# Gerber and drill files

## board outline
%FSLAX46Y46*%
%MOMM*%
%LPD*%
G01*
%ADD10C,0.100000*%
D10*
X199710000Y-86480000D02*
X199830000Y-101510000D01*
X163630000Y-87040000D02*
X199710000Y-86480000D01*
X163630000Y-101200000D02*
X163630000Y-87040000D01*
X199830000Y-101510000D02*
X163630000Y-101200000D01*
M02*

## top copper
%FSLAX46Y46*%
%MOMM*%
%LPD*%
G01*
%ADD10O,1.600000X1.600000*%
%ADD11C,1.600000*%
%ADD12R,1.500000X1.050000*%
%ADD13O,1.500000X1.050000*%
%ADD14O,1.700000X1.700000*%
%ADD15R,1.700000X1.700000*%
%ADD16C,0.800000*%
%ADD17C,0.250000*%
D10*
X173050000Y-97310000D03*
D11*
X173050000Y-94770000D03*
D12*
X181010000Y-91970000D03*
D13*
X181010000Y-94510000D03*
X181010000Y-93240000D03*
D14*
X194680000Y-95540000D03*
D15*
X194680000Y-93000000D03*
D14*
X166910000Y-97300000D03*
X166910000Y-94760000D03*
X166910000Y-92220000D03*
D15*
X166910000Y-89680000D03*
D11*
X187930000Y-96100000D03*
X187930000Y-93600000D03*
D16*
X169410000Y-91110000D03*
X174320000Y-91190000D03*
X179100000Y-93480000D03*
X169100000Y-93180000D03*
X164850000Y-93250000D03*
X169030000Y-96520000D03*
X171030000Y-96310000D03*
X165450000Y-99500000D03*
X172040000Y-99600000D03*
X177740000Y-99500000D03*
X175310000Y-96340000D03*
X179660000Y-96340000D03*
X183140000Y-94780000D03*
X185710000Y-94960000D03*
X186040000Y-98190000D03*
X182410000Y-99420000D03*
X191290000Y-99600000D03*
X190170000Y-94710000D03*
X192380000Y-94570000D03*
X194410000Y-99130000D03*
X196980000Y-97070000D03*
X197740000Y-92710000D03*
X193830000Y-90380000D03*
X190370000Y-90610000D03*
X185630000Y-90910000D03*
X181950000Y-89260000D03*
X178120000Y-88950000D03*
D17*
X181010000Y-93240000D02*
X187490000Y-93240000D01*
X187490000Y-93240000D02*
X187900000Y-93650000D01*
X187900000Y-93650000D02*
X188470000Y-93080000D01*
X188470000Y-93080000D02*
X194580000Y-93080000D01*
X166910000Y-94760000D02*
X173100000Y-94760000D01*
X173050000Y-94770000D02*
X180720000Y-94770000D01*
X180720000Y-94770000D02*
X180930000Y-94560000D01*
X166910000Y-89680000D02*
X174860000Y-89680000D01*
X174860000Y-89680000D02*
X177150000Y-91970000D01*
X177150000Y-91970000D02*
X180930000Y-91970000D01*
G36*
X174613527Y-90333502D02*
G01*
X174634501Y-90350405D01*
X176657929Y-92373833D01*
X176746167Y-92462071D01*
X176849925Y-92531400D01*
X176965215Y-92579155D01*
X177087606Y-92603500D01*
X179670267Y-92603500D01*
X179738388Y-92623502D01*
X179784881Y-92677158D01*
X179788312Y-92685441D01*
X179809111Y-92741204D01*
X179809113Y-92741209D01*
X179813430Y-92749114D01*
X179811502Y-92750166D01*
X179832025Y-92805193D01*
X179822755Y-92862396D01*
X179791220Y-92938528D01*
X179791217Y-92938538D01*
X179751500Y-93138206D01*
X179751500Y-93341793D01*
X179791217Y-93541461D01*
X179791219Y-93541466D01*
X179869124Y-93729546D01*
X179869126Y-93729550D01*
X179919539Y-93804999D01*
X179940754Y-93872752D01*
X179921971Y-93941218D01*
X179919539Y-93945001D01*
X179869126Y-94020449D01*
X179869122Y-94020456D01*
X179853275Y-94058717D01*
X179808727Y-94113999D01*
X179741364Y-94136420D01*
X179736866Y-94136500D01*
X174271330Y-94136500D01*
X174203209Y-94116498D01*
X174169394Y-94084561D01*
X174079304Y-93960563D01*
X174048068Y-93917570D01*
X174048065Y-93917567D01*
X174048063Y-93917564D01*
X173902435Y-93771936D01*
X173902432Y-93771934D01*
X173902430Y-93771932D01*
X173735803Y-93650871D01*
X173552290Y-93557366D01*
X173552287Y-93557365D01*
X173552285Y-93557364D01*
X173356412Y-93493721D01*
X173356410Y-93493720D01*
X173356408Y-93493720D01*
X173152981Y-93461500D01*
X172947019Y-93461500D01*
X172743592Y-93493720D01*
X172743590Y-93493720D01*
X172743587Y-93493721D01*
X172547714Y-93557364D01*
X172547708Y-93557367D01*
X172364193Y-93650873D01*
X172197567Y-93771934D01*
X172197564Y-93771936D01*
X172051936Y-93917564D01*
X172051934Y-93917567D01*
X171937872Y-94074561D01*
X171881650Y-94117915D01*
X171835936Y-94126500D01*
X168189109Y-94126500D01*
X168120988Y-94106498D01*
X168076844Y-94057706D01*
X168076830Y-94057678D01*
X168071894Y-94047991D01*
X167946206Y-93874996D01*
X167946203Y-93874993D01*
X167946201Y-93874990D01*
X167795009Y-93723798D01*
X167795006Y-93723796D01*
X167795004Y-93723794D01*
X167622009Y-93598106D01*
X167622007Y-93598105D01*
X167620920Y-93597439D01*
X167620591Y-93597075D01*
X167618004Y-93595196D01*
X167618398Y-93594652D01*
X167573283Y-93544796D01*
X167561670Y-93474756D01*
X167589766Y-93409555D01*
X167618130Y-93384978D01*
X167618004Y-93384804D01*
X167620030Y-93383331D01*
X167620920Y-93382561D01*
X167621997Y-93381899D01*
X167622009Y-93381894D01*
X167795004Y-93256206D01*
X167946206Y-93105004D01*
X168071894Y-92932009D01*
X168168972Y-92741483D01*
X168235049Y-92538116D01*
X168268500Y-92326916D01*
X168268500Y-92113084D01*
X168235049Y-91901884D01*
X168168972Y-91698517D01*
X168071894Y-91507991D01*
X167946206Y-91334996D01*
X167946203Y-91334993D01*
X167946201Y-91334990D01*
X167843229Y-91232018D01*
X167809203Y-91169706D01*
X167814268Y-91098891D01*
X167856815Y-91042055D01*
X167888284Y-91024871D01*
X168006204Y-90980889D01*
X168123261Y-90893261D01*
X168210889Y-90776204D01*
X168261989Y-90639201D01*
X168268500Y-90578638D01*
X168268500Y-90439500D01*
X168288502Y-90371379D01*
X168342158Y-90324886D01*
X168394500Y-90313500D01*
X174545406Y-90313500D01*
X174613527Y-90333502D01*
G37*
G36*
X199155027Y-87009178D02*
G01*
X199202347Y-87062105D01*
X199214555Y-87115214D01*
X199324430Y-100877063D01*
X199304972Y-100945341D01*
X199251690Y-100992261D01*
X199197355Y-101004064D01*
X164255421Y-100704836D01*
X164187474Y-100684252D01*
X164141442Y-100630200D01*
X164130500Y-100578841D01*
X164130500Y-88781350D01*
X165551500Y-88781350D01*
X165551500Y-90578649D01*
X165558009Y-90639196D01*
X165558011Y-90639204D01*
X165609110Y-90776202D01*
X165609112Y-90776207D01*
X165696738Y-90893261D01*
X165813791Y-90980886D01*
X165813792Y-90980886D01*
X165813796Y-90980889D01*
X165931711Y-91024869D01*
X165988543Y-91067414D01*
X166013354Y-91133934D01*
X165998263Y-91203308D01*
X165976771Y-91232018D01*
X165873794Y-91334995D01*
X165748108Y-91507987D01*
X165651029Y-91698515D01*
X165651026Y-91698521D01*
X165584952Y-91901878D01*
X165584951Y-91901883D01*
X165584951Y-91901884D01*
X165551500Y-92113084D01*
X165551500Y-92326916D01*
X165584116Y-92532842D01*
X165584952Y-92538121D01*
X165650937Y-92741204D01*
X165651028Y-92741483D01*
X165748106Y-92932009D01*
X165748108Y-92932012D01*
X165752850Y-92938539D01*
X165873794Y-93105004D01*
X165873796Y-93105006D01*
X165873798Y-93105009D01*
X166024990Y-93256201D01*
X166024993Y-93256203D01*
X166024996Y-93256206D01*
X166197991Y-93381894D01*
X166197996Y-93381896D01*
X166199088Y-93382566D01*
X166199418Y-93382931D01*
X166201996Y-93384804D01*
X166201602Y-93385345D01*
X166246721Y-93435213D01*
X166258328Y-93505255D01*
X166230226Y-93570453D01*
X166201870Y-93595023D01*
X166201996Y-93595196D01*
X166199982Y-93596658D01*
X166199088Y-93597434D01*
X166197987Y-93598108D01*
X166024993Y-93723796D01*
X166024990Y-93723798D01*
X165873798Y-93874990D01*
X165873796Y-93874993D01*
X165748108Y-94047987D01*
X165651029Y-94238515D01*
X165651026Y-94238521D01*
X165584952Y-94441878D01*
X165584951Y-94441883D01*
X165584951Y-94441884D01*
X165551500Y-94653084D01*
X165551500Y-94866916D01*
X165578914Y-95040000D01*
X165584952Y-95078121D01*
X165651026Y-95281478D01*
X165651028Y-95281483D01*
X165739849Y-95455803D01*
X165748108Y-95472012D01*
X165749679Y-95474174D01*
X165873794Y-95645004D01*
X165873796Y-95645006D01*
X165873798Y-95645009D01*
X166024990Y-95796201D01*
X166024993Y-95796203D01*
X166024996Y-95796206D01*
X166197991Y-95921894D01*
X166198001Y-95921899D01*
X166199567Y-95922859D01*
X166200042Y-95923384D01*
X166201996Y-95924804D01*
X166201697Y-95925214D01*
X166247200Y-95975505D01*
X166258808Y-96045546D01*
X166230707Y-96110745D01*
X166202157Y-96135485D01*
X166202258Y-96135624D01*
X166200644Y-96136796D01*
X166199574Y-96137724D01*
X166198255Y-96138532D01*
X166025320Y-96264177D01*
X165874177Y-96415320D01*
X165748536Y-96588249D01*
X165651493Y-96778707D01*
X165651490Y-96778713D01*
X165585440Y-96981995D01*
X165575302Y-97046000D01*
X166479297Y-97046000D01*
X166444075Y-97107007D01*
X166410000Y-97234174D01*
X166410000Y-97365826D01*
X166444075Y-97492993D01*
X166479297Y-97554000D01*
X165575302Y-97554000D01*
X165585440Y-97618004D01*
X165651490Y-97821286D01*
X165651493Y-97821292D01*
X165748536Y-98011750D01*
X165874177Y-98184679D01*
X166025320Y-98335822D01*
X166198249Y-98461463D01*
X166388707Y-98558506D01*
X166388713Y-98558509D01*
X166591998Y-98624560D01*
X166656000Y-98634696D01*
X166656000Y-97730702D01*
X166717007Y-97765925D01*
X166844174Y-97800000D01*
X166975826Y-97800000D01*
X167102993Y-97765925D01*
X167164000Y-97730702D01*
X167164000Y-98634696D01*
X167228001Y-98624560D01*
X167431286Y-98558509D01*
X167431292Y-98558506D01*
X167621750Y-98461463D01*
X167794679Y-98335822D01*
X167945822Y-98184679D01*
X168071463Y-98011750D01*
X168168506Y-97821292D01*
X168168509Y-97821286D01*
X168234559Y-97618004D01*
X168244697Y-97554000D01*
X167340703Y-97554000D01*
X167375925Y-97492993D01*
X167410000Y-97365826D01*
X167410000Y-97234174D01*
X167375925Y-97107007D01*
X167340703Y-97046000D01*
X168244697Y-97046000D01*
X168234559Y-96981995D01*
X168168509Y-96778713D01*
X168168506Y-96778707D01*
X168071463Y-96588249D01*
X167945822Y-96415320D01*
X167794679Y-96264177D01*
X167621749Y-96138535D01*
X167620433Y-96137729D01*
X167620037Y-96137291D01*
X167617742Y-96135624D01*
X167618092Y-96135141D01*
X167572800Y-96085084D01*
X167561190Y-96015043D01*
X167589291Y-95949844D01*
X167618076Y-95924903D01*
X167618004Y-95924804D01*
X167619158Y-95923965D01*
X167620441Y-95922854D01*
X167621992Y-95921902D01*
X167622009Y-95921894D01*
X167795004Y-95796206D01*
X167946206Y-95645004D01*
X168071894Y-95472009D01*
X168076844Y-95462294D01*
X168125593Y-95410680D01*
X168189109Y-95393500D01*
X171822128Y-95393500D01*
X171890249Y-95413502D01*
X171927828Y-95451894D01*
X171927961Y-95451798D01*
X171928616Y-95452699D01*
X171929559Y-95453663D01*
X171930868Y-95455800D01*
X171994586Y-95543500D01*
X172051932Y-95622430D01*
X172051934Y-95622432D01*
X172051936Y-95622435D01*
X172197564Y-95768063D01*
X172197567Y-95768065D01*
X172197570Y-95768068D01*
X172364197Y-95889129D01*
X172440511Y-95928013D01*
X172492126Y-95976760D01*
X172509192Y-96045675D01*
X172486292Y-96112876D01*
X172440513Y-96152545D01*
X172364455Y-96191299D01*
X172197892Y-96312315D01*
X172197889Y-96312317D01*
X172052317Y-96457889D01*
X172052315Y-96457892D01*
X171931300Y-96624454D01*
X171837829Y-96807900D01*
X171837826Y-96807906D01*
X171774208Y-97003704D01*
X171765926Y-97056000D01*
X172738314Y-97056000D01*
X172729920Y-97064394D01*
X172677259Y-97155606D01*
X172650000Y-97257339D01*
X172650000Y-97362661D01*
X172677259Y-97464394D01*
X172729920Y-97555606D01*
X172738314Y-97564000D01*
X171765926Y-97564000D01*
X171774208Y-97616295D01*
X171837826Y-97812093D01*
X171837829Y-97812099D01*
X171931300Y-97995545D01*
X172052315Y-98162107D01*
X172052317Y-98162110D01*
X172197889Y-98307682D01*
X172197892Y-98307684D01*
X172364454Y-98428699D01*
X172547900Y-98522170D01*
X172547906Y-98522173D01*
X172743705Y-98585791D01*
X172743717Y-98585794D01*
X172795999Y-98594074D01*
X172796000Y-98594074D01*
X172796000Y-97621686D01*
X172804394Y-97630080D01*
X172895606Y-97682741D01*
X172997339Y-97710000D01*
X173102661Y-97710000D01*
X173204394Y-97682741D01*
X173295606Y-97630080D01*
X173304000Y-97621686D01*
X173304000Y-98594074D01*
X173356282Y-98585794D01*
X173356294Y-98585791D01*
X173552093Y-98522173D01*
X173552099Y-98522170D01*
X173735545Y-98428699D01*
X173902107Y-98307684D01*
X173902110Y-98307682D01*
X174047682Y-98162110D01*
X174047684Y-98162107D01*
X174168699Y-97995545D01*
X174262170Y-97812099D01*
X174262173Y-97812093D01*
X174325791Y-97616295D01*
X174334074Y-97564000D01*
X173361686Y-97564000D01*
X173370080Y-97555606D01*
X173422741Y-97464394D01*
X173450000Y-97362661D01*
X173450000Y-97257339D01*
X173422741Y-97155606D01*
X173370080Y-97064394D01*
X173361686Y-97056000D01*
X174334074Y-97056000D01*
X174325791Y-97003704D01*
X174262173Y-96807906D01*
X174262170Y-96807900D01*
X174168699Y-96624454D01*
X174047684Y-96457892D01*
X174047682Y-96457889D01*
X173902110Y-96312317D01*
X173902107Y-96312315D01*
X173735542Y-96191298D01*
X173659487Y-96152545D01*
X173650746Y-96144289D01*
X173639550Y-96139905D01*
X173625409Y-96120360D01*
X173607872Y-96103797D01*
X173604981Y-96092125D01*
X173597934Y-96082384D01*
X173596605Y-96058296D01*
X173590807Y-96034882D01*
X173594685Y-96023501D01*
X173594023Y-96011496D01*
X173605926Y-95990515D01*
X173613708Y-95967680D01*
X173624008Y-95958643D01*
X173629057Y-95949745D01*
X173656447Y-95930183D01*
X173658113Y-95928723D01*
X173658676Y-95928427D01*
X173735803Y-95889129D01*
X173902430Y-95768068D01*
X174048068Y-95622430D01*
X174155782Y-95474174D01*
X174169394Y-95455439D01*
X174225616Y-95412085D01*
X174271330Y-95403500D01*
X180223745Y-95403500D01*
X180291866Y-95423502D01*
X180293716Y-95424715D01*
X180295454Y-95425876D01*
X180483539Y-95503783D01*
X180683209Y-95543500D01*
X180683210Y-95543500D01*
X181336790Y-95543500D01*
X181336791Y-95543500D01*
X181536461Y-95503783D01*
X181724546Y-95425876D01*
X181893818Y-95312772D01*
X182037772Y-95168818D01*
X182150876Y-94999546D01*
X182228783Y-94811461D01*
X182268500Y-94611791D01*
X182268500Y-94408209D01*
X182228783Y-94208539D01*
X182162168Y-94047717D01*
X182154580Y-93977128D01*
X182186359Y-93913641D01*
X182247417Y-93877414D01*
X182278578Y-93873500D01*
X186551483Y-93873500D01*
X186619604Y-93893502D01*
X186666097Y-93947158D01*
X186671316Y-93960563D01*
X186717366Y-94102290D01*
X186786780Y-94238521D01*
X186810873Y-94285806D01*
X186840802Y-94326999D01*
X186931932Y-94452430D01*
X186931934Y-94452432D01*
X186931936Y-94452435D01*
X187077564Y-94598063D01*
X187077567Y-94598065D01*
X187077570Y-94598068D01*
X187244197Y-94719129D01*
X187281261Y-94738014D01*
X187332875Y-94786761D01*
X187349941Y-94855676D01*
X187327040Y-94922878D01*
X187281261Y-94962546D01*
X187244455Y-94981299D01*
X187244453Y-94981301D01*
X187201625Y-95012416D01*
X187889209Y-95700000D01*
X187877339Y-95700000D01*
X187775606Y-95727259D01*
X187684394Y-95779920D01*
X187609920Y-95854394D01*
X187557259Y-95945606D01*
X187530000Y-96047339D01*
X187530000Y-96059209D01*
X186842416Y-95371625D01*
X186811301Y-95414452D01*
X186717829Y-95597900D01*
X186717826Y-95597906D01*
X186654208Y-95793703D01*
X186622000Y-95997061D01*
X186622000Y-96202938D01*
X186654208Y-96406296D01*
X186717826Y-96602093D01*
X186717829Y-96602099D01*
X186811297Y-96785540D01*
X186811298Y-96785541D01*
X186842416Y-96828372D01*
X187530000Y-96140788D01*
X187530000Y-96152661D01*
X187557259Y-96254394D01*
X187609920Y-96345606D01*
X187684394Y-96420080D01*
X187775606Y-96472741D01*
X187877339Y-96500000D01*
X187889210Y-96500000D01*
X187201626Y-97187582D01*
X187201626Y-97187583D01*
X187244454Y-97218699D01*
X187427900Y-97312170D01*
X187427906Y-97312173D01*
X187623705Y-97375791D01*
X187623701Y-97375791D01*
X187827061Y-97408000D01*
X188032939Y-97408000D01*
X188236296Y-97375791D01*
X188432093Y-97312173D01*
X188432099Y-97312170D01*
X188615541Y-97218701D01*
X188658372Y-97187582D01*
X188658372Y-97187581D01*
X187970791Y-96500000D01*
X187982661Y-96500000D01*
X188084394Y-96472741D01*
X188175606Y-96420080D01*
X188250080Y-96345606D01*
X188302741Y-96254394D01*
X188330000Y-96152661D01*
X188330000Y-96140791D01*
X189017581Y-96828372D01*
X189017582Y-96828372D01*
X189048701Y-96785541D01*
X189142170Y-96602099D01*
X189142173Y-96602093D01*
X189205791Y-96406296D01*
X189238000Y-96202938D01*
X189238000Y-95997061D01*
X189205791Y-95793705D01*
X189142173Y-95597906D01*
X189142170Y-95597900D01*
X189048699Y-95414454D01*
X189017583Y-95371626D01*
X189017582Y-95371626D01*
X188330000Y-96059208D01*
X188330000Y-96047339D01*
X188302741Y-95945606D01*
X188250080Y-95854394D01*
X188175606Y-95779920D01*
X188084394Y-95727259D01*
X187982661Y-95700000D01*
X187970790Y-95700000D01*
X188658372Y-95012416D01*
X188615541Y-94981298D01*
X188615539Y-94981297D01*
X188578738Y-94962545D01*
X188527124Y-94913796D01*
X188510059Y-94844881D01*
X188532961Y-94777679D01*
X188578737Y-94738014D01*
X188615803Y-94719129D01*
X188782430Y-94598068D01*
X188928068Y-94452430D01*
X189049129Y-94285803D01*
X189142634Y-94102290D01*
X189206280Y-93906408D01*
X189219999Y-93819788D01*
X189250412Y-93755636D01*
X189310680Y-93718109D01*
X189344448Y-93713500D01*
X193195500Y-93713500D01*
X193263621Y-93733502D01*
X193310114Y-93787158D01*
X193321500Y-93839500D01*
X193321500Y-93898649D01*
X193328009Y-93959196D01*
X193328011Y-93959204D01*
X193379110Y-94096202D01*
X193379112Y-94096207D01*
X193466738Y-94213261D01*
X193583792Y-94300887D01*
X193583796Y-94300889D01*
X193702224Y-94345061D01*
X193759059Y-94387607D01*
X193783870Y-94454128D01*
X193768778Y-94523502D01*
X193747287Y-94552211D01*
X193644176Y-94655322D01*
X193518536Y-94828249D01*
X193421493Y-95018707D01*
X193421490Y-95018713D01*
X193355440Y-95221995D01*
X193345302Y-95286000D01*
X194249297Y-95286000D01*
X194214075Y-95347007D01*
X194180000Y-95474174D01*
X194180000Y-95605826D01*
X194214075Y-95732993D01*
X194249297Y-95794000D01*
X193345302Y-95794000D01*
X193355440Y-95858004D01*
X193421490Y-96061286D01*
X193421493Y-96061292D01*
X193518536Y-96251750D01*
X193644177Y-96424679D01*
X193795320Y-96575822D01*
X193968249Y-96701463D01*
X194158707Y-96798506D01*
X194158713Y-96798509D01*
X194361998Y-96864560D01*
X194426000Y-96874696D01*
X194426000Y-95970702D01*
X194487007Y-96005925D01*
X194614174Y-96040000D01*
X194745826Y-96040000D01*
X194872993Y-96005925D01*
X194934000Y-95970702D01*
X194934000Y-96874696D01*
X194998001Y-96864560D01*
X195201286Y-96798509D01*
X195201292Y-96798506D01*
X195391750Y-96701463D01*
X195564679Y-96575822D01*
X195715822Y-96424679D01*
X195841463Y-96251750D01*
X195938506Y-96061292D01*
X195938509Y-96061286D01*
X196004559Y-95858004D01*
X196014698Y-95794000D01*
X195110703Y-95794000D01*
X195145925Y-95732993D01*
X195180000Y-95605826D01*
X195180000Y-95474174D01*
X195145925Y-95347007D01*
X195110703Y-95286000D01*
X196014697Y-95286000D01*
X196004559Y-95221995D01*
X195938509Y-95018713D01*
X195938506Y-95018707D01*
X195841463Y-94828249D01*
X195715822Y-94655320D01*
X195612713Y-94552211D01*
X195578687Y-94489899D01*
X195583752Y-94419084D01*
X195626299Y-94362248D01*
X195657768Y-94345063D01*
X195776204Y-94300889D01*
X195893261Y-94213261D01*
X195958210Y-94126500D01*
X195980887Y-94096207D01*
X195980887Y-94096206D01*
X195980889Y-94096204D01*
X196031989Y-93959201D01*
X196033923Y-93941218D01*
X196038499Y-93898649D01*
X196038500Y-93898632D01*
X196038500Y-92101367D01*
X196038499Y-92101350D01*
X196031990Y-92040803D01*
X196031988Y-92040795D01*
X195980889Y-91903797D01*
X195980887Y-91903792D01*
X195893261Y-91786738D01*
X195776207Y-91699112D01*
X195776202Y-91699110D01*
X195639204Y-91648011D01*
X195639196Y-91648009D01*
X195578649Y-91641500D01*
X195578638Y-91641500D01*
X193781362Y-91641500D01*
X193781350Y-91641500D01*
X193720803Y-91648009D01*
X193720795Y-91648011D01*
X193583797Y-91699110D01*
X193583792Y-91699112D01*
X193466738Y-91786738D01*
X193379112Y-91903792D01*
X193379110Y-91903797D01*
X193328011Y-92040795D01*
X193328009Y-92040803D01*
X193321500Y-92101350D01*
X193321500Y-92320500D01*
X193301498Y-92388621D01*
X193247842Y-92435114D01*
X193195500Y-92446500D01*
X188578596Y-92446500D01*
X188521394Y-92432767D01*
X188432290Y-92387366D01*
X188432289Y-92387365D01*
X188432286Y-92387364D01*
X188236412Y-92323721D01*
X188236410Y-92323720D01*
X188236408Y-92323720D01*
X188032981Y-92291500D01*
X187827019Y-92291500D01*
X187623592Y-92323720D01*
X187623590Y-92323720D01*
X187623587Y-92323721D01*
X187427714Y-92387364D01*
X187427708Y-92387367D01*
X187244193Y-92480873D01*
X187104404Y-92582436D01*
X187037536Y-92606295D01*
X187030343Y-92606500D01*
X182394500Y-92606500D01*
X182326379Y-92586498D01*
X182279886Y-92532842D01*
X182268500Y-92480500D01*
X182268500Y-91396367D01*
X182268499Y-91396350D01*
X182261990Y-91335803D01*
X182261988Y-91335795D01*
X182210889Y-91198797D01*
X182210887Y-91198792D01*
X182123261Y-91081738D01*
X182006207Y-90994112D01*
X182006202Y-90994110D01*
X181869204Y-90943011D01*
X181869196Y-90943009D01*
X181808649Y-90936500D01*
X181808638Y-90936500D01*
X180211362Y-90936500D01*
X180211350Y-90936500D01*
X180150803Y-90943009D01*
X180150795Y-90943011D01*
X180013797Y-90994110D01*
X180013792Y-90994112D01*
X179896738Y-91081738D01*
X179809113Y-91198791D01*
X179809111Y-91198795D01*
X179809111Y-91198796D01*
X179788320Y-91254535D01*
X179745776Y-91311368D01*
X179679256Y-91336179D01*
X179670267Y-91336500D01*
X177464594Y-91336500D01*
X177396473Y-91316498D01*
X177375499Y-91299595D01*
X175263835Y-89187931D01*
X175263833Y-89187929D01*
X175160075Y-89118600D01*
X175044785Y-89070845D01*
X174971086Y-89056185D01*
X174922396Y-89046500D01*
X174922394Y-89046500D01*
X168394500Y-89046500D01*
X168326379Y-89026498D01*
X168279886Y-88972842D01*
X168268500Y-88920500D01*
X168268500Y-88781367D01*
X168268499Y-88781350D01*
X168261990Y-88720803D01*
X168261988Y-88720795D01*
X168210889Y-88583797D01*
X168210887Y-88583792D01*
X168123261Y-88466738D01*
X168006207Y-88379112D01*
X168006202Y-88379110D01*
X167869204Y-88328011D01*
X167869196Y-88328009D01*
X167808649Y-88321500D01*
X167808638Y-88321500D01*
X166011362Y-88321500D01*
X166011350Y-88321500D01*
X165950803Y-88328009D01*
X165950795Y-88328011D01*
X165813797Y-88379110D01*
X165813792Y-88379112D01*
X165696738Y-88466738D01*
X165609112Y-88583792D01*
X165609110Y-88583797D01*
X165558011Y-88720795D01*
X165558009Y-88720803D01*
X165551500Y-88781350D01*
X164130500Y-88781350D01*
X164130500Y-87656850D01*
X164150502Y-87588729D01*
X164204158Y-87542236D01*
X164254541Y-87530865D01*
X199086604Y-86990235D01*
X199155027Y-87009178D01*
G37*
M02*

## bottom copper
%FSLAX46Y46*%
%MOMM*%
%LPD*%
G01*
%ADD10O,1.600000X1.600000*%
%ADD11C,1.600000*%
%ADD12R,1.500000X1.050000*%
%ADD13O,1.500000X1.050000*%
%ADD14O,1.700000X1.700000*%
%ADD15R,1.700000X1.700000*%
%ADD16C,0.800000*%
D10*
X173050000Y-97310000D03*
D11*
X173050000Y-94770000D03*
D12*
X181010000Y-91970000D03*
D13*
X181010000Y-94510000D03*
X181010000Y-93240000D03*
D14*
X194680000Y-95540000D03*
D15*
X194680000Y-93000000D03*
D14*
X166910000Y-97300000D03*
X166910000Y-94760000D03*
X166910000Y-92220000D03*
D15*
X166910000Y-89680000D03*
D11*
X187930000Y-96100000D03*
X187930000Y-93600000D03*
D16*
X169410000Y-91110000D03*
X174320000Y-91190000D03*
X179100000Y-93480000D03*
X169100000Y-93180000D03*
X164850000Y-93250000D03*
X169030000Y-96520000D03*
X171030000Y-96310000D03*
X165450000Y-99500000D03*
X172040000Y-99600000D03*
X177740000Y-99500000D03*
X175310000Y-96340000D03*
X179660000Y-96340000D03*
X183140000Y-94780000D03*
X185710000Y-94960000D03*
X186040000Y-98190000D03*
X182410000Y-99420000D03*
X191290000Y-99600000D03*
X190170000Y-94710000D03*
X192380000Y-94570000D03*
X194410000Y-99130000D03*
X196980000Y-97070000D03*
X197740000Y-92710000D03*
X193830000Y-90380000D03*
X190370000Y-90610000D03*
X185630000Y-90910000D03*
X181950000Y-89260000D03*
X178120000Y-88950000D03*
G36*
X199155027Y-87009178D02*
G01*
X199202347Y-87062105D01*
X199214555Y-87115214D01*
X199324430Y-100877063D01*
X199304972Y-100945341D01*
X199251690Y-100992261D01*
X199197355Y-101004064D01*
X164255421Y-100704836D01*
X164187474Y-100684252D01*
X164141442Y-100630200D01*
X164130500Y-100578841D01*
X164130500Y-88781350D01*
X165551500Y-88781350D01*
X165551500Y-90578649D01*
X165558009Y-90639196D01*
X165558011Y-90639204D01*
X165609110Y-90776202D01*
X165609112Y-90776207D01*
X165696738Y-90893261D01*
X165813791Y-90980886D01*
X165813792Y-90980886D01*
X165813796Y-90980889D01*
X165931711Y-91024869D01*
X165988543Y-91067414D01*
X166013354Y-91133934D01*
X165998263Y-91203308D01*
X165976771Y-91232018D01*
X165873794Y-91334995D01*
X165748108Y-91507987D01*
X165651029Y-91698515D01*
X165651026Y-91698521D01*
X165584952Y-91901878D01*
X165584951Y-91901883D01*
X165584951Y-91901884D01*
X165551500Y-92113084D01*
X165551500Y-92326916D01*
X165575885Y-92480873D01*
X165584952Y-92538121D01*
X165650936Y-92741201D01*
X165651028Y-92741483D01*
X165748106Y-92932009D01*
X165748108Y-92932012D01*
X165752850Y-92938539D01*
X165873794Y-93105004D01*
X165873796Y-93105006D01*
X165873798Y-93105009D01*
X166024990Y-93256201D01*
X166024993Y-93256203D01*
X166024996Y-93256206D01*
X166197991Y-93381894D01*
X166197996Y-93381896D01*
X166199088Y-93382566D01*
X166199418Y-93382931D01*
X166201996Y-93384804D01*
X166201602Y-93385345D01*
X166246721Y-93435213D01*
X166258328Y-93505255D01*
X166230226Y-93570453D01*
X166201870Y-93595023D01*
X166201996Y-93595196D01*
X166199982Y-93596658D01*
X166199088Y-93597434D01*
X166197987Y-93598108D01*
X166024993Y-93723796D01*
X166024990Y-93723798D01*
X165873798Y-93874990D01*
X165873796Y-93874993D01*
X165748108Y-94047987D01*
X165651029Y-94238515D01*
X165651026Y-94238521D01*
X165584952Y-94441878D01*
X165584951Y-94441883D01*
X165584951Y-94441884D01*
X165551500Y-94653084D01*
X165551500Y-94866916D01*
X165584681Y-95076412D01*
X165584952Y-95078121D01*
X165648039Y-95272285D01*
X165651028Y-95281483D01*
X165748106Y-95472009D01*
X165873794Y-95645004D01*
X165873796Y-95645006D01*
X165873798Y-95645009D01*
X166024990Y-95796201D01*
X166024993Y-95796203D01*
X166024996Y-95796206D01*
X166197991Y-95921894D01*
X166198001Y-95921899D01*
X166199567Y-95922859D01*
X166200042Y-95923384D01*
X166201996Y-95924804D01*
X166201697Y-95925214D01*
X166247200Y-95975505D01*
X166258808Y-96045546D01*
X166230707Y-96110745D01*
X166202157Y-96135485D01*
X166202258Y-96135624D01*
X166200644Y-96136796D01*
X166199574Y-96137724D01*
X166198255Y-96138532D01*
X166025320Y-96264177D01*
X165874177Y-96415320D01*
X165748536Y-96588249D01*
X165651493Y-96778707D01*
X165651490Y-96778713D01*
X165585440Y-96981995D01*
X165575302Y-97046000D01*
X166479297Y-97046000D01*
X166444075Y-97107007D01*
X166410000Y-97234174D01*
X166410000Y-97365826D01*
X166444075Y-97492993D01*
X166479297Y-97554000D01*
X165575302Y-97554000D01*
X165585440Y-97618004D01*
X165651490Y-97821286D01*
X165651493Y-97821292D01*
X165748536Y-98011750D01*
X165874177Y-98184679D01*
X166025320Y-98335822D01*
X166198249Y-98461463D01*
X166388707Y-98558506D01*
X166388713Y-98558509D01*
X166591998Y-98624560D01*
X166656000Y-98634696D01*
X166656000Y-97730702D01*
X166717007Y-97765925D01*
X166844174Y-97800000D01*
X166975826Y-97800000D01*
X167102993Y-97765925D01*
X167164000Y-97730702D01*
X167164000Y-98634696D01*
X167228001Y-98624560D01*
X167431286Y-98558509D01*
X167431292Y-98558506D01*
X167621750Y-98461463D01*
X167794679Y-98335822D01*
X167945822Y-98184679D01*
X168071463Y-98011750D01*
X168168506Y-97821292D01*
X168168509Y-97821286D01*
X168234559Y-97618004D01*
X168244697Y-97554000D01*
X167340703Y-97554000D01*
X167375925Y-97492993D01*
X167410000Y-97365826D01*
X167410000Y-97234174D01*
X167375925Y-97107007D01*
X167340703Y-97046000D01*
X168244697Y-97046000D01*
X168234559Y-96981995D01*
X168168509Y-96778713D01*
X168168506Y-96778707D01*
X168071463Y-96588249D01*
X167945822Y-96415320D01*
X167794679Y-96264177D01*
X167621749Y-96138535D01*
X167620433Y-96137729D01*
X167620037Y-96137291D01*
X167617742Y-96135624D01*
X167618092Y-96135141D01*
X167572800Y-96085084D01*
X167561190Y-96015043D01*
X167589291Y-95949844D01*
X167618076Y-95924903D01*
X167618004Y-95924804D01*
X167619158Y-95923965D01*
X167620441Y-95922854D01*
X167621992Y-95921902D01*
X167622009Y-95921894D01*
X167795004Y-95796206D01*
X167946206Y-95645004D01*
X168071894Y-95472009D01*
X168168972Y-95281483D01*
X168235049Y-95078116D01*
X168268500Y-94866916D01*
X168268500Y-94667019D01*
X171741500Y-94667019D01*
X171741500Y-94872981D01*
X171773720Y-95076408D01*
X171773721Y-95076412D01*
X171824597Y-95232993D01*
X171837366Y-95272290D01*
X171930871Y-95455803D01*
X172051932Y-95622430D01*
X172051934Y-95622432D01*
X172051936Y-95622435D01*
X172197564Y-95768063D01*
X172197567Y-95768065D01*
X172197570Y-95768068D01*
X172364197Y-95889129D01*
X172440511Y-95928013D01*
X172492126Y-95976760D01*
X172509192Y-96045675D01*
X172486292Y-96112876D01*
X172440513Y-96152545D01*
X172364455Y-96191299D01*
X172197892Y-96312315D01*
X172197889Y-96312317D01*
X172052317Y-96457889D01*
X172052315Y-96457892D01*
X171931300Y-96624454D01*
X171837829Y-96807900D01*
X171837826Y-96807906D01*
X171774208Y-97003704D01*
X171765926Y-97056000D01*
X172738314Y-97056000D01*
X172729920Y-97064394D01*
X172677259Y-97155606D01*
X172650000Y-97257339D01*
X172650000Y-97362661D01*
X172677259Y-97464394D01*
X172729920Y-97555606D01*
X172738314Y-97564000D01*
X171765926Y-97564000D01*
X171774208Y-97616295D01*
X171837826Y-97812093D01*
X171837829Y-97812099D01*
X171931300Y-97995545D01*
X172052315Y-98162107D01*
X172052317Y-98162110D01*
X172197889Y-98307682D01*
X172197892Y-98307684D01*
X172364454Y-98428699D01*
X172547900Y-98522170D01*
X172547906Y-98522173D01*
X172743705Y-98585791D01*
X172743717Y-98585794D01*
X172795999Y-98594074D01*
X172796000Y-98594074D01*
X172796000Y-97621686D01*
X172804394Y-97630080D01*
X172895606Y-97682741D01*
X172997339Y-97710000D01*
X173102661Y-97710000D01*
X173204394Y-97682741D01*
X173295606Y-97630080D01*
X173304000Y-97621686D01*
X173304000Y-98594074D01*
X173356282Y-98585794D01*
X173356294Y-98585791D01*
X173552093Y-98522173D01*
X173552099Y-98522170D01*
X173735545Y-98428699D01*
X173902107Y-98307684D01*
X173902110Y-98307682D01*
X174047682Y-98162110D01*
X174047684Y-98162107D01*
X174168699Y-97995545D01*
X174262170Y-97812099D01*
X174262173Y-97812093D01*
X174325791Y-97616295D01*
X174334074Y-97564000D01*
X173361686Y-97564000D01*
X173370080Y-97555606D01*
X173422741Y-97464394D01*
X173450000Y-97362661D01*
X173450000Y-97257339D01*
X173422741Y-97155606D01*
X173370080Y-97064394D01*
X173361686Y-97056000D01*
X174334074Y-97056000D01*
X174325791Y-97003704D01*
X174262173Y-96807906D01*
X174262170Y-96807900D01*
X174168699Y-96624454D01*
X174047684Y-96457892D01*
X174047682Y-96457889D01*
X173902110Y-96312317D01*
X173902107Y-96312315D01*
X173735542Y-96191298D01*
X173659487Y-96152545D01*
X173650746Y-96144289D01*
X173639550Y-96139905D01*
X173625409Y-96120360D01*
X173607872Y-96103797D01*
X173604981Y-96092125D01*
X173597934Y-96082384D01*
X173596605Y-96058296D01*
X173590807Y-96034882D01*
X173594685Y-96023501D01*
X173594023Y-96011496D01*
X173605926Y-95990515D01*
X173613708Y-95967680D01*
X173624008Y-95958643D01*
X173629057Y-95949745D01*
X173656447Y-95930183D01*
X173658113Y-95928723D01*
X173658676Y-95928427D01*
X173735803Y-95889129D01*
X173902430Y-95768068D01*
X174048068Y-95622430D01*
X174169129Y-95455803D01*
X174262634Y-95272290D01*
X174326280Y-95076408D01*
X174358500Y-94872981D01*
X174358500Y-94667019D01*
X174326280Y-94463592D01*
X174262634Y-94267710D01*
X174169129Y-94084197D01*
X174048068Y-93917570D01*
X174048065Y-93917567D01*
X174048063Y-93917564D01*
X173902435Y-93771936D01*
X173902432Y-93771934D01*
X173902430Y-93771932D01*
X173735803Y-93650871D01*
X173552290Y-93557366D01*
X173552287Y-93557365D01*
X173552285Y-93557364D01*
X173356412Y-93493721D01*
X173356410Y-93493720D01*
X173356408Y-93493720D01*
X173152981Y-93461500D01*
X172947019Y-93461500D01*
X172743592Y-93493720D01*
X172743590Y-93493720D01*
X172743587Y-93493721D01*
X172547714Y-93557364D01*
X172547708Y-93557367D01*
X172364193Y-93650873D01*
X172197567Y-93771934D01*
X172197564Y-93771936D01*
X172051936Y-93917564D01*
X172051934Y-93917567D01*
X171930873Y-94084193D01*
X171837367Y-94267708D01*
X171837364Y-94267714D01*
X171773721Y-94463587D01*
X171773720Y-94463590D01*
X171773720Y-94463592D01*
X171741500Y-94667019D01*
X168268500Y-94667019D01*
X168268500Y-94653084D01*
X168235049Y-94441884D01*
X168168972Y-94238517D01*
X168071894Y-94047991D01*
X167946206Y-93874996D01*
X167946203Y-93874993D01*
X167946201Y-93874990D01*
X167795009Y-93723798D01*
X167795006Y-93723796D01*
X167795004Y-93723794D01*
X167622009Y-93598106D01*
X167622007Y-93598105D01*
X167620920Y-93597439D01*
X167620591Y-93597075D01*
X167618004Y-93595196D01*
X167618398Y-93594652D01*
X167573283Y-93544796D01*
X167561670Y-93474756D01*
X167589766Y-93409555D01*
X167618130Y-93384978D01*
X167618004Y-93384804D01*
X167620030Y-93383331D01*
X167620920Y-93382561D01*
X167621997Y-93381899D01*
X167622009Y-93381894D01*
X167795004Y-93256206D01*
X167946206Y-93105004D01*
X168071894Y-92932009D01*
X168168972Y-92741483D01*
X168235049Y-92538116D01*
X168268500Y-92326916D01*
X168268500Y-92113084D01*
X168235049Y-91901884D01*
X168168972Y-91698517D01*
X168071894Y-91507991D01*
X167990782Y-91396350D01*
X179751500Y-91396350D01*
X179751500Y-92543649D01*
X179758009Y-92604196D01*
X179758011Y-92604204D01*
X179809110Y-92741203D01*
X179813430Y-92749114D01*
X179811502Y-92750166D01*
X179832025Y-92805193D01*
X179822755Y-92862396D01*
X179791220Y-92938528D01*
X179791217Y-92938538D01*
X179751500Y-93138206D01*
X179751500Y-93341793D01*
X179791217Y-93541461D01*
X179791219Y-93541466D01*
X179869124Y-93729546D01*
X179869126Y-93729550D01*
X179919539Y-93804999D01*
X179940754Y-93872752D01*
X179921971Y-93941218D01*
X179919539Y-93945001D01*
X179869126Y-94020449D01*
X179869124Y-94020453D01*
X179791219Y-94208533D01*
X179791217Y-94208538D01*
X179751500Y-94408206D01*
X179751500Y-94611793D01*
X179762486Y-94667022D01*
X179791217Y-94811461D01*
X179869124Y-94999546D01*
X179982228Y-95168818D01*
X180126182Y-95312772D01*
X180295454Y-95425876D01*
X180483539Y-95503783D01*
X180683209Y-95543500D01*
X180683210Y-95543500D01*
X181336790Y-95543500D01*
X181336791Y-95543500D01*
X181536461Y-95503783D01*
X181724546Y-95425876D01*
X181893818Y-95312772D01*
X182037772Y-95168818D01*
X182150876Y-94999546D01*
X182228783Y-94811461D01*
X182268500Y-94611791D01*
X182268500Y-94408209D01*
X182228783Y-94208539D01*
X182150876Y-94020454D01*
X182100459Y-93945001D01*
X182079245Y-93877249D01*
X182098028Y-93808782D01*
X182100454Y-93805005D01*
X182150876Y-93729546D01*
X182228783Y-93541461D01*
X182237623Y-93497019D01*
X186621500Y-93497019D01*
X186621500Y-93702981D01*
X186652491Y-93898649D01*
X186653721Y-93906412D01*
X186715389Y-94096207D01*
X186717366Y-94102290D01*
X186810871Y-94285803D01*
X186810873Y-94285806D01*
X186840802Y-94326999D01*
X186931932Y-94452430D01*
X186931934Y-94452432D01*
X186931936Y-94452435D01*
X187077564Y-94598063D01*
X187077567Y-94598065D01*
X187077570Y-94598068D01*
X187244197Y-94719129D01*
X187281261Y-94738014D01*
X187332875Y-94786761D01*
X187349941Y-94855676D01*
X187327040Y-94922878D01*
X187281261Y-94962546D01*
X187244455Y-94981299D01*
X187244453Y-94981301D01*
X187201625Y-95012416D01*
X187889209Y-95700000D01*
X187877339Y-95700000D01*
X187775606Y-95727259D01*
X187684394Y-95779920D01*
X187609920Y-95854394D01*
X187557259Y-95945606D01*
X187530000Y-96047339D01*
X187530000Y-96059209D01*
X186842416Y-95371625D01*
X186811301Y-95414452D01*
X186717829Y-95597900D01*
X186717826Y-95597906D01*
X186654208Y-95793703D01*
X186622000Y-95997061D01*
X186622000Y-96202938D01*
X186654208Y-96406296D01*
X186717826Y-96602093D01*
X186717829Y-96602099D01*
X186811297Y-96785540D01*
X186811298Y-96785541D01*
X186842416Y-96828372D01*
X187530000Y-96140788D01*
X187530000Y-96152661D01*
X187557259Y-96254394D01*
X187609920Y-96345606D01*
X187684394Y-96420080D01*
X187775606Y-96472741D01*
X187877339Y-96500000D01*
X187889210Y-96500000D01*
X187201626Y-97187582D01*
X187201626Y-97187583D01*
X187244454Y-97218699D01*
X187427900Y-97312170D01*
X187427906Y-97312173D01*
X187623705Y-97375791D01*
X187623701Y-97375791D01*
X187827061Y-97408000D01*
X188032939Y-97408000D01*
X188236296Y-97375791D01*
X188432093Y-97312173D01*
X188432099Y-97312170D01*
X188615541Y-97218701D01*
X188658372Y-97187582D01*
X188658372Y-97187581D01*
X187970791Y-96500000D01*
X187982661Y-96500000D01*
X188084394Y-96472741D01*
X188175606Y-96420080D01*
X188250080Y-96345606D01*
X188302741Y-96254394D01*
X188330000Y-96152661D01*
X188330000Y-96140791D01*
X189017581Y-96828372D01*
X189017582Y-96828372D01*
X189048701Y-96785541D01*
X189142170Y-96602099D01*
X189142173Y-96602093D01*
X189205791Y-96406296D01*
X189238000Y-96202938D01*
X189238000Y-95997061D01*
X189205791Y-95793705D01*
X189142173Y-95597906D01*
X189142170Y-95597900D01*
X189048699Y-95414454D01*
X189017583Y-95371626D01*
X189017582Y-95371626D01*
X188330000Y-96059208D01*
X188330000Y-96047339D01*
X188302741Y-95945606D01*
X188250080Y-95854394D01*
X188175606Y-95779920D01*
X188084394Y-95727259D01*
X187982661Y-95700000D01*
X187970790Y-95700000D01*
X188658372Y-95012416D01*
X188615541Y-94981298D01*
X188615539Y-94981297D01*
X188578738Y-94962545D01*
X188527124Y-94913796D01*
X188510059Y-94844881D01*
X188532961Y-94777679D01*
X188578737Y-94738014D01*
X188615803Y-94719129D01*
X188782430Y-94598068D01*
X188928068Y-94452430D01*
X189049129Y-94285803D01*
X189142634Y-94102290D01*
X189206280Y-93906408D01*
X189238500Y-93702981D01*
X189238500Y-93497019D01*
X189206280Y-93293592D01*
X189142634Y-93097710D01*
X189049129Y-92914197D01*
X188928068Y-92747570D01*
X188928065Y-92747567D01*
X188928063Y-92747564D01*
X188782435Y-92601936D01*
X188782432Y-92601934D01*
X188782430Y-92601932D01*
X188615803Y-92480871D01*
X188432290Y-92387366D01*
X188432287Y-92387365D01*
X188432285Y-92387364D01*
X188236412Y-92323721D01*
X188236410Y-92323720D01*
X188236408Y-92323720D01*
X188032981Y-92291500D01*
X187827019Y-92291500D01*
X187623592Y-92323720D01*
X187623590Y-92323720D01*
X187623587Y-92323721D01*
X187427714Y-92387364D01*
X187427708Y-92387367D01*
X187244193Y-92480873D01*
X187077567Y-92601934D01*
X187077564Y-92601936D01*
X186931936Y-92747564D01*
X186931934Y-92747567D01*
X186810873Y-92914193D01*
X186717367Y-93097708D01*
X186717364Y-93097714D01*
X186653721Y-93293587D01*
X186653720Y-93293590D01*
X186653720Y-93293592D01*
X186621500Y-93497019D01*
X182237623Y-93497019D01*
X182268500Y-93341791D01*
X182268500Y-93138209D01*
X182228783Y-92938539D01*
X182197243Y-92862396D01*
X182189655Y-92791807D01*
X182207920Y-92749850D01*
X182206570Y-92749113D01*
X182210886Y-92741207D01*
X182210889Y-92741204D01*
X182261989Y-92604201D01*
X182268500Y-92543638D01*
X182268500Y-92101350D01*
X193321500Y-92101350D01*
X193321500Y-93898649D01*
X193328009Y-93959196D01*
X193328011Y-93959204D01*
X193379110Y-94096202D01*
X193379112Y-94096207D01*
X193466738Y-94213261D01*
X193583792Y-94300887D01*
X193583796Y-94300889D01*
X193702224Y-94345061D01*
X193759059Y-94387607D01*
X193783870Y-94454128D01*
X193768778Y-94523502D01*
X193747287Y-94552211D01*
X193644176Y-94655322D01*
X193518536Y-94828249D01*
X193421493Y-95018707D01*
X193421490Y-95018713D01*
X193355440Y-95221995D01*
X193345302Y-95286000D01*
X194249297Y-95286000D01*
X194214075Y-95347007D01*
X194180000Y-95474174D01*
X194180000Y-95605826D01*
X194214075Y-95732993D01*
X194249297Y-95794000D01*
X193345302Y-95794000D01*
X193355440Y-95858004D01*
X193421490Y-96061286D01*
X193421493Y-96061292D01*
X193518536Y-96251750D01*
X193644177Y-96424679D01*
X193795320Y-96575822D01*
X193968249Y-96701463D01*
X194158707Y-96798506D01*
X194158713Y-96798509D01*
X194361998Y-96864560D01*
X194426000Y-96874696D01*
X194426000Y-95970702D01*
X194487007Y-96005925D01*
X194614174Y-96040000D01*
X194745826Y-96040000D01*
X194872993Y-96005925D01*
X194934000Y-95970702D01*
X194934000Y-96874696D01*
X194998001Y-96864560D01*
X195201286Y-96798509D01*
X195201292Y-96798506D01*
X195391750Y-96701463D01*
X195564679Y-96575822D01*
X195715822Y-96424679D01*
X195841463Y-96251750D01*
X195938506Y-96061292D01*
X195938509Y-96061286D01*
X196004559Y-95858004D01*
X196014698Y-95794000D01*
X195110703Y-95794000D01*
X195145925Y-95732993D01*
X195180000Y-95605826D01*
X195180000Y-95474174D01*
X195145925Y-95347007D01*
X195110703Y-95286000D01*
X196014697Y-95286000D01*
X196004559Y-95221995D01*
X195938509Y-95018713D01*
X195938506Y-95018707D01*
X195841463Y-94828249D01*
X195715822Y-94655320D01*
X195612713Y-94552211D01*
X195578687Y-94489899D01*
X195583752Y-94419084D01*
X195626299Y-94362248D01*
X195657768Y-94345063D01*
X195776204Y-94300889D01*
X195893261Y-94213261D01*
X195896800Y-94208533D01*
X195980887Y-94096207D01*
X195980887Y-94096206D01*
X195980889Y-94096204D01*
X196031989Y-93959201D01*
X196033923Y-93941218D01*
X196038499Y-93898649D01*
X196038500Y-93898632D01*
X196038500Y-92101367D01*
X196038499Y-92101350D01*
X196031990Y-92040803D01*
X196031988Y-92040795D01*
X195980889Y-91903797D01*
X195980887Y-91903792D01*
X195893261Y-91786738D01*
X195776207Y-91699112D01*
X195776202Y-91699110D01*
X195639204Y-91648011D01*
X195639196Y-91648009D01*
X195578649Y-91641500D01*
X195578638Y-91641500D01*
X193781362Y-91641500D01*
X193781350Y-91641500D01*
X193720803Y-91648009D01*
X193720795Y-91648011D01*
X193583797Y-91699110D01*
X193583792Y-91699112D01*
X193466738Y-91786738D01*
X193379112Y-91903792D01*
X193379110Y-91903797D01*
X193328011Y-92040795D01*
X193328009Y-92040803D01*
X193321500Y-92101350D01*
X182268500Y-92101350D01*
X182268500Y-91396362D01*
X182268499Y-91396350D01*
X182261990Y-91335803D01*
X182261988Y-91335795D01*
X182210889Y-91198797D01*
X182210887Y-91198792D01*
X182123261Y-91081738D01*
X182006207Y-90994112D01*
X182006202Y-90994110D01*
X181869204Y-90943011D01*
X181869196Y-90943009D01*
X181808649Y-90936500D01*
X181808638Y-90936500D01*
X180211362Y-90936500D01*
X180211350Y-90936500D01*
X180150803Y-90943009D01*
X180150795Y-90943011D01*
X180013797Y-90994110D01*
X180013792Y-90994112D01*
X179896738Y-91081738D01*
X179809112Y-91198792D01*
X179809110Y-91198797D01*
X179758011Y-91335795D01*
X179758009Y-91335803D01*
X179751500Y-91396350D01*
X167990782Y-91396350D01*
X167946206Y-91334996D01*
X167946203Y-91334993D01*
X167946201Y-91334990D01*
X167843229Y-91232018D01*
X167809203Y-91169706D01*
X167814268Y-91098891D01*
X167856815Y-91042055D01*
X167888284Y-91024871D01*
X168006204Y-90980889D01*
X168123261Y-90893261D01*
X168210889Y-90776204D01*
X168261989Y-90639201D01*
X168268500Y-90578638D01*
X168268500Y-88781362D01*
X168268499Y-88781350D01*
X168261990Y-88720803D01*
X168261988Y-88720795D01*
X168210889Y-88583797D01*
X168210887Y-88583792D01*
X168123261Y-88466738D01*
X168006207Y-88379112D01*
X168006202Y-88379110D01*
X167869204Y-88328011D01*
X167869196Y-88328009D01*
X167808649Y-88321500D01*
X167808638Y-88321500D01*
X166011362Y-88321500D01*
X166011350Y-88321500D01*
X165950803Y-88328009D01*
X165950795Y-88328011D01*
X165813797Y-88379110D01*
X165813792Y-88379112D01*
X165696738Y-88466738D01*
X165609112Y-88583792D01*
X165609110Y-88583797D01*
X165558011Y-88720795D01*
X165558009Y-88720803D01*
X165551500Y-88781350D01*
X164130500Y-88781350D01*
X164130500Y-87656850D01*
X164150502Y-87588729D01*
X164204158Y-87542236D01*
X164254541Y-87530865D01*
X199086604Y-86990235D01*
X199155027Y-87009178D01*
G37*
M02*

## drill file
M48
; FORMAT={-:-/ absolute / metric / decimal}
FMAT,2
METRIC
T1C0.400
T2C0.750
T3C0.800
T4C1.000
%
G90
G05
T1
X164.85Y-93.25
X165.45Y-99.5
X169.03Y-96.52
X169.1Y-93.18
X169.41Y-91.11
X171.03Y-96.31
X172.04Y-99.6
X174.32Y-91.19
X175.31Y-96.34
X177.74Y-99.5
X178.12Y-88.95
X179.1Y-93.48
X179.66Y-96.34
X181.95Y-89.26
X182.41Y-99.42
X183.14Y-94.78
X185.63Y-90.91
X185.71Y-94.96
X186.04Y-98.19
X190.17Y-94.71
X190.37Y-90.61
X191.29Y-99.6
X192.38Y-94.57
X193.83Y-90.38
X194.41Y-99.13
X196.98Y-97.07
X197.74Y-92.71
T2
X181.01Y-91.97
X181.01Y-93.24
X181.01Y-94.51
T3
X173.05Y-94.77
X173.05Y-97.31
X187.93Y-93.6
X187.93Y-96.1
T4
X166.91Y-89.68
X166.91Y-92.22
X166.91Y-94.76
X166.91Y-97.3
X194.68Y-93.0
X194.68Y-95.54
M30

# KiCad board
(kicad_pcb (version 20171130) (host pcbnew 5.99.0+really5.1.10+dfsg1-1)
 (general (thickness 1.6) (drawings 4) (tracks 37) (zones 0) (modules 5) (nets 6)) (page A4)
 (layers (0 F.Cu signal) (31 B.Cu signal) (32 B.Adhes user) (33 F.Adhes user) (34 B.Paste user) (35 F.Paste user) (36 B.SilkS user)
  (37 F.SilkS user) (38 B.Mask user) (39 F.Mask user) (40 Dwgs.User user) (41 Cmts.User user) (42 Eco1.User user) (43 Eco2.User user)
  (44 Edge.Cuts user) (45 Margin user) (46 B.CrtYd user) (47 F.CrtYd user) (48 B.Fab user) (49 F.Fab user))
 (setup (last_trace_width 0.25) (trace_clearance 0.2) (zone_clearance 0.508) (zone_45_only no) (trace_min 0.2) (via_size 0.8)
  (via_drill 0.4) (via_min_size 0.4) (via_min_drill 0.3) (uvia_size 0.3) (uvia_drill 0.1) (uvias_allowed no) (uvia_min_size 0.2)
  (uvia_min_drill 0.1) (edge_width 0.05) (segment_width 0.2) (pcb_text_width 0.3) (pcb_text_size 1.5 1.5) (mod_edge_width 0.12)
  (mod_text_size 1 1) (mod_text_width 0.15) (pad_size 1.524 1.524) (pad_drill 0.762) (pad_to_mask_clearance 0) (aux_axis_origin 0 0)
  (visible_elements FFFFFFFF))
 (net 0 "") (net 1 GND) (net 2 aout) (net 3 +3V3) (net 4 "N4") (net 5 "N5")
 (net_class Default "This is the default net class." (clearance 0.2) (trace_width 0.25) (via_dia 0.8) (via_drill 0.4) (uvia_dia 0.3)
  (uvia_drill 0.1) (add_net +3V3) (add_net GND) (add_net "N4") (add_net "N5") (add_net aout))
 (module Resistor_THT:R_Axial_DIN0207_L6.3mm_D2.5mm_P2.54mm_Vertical (layer F.Cu) (at 173.05 94.77 270)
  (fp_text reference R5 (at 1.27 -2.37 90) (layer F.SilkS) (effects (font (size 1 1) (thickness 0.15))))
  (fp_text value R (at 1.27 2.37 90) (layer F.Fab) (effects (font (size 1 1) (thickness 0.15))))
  (pad 2 thru_hole oval (at 2.54 0 270) (size 1.6 1.6) (drill 0.8) (layers *.Cu *.Mask) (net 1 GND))
  (pad 1 thru_hole circle (at 0 0 270) (size 1.6 1.6) (drill 0.8) (layers *.Cu *.Mask) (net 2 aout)))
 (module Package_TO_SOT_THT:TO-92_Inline (layer F.Cu) (at 181.01 91.97 270)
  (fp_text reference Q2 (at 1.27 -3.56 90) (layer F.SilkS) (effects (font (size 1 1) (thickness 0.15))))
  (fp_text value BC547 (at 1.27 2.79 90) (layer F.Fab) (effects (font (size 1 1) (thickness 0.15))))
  (pad 1 thru_hole rect (at 0 0 270) (size 1.05 1.5) (drill 0.75) (layers *.Cu *.Mask) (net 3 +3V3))
  (pad 3 thru_hole oval (at 2.54 0 270) (size 1.05 1.5) (drill 0.75) (layers *.Cu *.Mask) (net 2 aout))
  (pad 2 thru_hole oval (at 1.27 0 270) (size 1.05 1.5) (drill 0.75) (layers *.Cu *.Mask) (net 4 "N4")))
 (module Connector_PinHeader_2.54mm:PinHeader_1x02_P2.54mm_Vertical (layer F.Cu) (at 194.68 93)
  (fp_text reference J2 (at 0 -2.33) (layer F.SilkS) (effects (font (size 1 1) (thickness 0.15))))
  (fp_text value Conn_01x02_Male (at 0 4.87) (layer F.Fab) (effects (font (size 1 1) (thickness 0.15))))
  (pad 2 thru_hole oval (at 0 2.54) (size 1.7 1.7) (drill 1) (layers *.Cu *.Mask) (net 1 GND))
  (pad 1 thru_hole rect (at 0 0) (size 1.7 1.7) (drill 1) (layers *.Cu *.Mask) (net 4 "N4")))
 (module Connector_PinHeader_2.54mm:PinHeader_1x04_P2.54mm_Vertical (layer F.Cu) (at 166.91 89.68)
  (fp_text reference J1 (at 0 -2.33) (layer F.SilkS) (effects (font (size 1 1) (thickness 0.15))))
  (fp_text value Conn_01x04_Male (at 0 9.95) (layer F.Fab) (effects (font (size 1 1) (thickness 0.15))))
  (pad 4 thru_hole oval (at 0 7.62) (size 1.7 1.7) (drill 1) (layers *.Cu *.Mask) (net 1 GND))
  (pad 3 thru_hole oval (at 0 5.08) (size 1.7 1.7) (drill 1) (layers *.Cu *.Mask) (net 2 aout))
  (pad 2 thru_hole oval (at 0 2.54) (size 1.7 1.7) (drill 1) (layers *.Cu *.Mask) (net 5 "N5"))
  (pad 1 thru_hole rect (at 0 0) (size 1.7 1.7) (drill 1) (layers *.Cu *.Mask) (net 3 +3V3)))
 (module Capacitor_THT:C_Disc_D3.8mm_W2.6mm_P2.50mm (layer F.Cu) (at 187.93 93.6 270)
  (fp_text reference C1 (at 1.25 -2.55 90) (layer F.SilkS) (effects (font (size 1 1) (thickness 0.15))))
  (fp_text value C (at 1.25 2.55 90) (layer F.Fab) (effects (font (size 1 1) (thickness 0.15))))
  (pad 2 thru_hole circle (at 2.5 0 270) (size 1.6 1.6) (drill 0.8) (layers *.Cu *.Mask) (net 1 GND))
  (pad 1 thru_hole circle (at 0 0 270) (size 1.6 1.6) (drill 0.8) (layers *.Cu *.Mask) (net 4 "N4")))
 (gr_line (start 199.71 86.48) (end 199.83 101.51) (layer Edge.Cuts) (width 0.1))
 (gr_line (start 163.63 87.04) (end 199.71 86.48) (layer Edge.Cuts) (width 0.1))
 (gr_line (start 163.63 101.2) (end 163.63 87.04) (layer Edge.Cuts) (width 0.1))
 (gr_line (start 199.83 101.51) (end 163.63 101.2) (layer Edge.Cuts) (width 0.1))
 (via (at 169.41 91.11) (size 0.8) (drill 0.4) (layers F.Cu B.Cu) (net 1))
 (via (at 174.32 91.19) (size 0.8) (drill 0.4) (layers F.Cu B.Cu) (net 1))
 (via (at 179.1 93.48) (size 0.8) (drill 0.4) (layers F.Cu B.Cu) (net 1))
 (via (at 169.1 93.18) (size 0.8) (drill 0.4) (layers F.Cu B.Cu) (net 1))
 (via (at 164.85 93.25) (size 0.8) (drill 0.4) (layers F.Cu B.Cu) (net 1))
 (via (at 169.03 96.52) (size 0.8) (drill 0.4) (layers F.Cu B.Cu) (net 1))
 (via (at 171.03 96.31) (size 0.8) (drill 0.4) (layers F.Cu B.Cu) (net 1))
 (via (at 165.45 99.5) (size 0.8) (drill 0.4) (layers F.Cu B.Cu) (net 1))
 (via (at 172.04 99.6) (size 0.8) (drill 0.4) (layers F.Cu B.Cu) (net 1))
 (via (at 177.74 99.5) (size 0.8) (drill 0.4) (layers F.Cu B.Cu) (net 1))
 (via (at 175.31 96.34) (size 0.8) (drill 0.4) (layers F.Cu B.Cu) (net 1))
 (via (at 179.66 96.34) (size 0.8) (drill 0.4) (layers F.Cu B.Cu) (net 1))
 (via (at 183.14 94.78) (size 0.8) (drill 0.4) (layers F.Cu B.Cu) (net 1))
 (via (at 185.71 94.96) (size 0.8) (drill 0.4) (layers F.Cu B.Cu) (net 1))
 (via (at 186.04 98.19) (size 0.8) (drill 0.4) (layers F.Cu B.Cu) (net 1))
 (via (at 182.41 99.42) (size 0.8) (drill 0.4) (layers F.Cu B.Cu) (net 1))
 (via (at 191.29 99.6) (size 0.8) (drill 0.4) (layers F.Cu B.Cu) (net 1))
 (via (at 190.17 94.71) (size 0.8) (drill 0.4) (layers F.Cu B.Cu) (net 1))
 (via (at 192.38 94.57) (size 0.8) (drill 0.4) (layers F.Cu B.Cu) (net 1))
 (via (at 194.41 99.13) (size 0.8) (drill 0.4) (layers F.Cu B.Cu) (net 1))
 (via (at 196.98 97.07) (size 0.8) (drill 0.4) (layers F.Cu B.Cu) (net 1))
 (via (at 197.74 92.71) (size 0.8) (drill 0.4) (layers F.Cu B.Cu) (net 1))
 (via (at 193.83 90.38) (size 0.8) (drill 0.4) (layers F.Cu B.Cu) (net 1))
 (via (at 190.37 90.61) (size 0.8) (drill 0.4) (layers F.Cu B.Cu) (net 1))
 (via (at 185.63 90.91) (size 0.8) (drill 0.4) (layers F.Cu B.Cu) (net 1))
 (via (at 181.95 89.26) (size 0.8) (drill 0.4) (layers F.Cu B.Cu) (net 1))
 (via (at 178.12 88.95) (size 0.8) (drill 0.4) (layers F.Cu B.Cu) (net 1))
 (segment (start 181.01 93.24) (end 187.49 93.24) (width 0.25) (layer F.Cu) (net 4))
 (segment (start 187.49 93.24) (end 187.9 93.65) (width 0.25) (layer F.Cu) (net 4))
 (segment (start 187.9 93.65) (end 188.47 93.08) (width 0.25) (layer F.Cu) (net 4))
 (segment (start 188.47 93.08) (end 194.58 93.08) (width 0.25) (layer F.Cu) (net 4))
 (segment (start 166.91 94.76) (end 173.1 94.76) (width 0.25) (layer F.Cu) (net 2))
 (segment (start 173.05 94.77) (end 180.72 94.77) (width 0.25) (layer F.Cu) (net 2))
 (segment (start 180.72 94.77) (end 180.93 94.56) (width 0.25) (layer F.Cu) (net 2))
 (segment (start 166.91 89.68) (end 174.86 89.68) (width 0.25) (layer F.Cu) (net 3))
 (segment (start 174.86 89.68) (end 177.15 91.97) (width 0.25) (layer F.Cu) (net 3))
 (segment (start 177.15 91.97) (end 180.93 91.97) (width 0.25) (layer F.Cu) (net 3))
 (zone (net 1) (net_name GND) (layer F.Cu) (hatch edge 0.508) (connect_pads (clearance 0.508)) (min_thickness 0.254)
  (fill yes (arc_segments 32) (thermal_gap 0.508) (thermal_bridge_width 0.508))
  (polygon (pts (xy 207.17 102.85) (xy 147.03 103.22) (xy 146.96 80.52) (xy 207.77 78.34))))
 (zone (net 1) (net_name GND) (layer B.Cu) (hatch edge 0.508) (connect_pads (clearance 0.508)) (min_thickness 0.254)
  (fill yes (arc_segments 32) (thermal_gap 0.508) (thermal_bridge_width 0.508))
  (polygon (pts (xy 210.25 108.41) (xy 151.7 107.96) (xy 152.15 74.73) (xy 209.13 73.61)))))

